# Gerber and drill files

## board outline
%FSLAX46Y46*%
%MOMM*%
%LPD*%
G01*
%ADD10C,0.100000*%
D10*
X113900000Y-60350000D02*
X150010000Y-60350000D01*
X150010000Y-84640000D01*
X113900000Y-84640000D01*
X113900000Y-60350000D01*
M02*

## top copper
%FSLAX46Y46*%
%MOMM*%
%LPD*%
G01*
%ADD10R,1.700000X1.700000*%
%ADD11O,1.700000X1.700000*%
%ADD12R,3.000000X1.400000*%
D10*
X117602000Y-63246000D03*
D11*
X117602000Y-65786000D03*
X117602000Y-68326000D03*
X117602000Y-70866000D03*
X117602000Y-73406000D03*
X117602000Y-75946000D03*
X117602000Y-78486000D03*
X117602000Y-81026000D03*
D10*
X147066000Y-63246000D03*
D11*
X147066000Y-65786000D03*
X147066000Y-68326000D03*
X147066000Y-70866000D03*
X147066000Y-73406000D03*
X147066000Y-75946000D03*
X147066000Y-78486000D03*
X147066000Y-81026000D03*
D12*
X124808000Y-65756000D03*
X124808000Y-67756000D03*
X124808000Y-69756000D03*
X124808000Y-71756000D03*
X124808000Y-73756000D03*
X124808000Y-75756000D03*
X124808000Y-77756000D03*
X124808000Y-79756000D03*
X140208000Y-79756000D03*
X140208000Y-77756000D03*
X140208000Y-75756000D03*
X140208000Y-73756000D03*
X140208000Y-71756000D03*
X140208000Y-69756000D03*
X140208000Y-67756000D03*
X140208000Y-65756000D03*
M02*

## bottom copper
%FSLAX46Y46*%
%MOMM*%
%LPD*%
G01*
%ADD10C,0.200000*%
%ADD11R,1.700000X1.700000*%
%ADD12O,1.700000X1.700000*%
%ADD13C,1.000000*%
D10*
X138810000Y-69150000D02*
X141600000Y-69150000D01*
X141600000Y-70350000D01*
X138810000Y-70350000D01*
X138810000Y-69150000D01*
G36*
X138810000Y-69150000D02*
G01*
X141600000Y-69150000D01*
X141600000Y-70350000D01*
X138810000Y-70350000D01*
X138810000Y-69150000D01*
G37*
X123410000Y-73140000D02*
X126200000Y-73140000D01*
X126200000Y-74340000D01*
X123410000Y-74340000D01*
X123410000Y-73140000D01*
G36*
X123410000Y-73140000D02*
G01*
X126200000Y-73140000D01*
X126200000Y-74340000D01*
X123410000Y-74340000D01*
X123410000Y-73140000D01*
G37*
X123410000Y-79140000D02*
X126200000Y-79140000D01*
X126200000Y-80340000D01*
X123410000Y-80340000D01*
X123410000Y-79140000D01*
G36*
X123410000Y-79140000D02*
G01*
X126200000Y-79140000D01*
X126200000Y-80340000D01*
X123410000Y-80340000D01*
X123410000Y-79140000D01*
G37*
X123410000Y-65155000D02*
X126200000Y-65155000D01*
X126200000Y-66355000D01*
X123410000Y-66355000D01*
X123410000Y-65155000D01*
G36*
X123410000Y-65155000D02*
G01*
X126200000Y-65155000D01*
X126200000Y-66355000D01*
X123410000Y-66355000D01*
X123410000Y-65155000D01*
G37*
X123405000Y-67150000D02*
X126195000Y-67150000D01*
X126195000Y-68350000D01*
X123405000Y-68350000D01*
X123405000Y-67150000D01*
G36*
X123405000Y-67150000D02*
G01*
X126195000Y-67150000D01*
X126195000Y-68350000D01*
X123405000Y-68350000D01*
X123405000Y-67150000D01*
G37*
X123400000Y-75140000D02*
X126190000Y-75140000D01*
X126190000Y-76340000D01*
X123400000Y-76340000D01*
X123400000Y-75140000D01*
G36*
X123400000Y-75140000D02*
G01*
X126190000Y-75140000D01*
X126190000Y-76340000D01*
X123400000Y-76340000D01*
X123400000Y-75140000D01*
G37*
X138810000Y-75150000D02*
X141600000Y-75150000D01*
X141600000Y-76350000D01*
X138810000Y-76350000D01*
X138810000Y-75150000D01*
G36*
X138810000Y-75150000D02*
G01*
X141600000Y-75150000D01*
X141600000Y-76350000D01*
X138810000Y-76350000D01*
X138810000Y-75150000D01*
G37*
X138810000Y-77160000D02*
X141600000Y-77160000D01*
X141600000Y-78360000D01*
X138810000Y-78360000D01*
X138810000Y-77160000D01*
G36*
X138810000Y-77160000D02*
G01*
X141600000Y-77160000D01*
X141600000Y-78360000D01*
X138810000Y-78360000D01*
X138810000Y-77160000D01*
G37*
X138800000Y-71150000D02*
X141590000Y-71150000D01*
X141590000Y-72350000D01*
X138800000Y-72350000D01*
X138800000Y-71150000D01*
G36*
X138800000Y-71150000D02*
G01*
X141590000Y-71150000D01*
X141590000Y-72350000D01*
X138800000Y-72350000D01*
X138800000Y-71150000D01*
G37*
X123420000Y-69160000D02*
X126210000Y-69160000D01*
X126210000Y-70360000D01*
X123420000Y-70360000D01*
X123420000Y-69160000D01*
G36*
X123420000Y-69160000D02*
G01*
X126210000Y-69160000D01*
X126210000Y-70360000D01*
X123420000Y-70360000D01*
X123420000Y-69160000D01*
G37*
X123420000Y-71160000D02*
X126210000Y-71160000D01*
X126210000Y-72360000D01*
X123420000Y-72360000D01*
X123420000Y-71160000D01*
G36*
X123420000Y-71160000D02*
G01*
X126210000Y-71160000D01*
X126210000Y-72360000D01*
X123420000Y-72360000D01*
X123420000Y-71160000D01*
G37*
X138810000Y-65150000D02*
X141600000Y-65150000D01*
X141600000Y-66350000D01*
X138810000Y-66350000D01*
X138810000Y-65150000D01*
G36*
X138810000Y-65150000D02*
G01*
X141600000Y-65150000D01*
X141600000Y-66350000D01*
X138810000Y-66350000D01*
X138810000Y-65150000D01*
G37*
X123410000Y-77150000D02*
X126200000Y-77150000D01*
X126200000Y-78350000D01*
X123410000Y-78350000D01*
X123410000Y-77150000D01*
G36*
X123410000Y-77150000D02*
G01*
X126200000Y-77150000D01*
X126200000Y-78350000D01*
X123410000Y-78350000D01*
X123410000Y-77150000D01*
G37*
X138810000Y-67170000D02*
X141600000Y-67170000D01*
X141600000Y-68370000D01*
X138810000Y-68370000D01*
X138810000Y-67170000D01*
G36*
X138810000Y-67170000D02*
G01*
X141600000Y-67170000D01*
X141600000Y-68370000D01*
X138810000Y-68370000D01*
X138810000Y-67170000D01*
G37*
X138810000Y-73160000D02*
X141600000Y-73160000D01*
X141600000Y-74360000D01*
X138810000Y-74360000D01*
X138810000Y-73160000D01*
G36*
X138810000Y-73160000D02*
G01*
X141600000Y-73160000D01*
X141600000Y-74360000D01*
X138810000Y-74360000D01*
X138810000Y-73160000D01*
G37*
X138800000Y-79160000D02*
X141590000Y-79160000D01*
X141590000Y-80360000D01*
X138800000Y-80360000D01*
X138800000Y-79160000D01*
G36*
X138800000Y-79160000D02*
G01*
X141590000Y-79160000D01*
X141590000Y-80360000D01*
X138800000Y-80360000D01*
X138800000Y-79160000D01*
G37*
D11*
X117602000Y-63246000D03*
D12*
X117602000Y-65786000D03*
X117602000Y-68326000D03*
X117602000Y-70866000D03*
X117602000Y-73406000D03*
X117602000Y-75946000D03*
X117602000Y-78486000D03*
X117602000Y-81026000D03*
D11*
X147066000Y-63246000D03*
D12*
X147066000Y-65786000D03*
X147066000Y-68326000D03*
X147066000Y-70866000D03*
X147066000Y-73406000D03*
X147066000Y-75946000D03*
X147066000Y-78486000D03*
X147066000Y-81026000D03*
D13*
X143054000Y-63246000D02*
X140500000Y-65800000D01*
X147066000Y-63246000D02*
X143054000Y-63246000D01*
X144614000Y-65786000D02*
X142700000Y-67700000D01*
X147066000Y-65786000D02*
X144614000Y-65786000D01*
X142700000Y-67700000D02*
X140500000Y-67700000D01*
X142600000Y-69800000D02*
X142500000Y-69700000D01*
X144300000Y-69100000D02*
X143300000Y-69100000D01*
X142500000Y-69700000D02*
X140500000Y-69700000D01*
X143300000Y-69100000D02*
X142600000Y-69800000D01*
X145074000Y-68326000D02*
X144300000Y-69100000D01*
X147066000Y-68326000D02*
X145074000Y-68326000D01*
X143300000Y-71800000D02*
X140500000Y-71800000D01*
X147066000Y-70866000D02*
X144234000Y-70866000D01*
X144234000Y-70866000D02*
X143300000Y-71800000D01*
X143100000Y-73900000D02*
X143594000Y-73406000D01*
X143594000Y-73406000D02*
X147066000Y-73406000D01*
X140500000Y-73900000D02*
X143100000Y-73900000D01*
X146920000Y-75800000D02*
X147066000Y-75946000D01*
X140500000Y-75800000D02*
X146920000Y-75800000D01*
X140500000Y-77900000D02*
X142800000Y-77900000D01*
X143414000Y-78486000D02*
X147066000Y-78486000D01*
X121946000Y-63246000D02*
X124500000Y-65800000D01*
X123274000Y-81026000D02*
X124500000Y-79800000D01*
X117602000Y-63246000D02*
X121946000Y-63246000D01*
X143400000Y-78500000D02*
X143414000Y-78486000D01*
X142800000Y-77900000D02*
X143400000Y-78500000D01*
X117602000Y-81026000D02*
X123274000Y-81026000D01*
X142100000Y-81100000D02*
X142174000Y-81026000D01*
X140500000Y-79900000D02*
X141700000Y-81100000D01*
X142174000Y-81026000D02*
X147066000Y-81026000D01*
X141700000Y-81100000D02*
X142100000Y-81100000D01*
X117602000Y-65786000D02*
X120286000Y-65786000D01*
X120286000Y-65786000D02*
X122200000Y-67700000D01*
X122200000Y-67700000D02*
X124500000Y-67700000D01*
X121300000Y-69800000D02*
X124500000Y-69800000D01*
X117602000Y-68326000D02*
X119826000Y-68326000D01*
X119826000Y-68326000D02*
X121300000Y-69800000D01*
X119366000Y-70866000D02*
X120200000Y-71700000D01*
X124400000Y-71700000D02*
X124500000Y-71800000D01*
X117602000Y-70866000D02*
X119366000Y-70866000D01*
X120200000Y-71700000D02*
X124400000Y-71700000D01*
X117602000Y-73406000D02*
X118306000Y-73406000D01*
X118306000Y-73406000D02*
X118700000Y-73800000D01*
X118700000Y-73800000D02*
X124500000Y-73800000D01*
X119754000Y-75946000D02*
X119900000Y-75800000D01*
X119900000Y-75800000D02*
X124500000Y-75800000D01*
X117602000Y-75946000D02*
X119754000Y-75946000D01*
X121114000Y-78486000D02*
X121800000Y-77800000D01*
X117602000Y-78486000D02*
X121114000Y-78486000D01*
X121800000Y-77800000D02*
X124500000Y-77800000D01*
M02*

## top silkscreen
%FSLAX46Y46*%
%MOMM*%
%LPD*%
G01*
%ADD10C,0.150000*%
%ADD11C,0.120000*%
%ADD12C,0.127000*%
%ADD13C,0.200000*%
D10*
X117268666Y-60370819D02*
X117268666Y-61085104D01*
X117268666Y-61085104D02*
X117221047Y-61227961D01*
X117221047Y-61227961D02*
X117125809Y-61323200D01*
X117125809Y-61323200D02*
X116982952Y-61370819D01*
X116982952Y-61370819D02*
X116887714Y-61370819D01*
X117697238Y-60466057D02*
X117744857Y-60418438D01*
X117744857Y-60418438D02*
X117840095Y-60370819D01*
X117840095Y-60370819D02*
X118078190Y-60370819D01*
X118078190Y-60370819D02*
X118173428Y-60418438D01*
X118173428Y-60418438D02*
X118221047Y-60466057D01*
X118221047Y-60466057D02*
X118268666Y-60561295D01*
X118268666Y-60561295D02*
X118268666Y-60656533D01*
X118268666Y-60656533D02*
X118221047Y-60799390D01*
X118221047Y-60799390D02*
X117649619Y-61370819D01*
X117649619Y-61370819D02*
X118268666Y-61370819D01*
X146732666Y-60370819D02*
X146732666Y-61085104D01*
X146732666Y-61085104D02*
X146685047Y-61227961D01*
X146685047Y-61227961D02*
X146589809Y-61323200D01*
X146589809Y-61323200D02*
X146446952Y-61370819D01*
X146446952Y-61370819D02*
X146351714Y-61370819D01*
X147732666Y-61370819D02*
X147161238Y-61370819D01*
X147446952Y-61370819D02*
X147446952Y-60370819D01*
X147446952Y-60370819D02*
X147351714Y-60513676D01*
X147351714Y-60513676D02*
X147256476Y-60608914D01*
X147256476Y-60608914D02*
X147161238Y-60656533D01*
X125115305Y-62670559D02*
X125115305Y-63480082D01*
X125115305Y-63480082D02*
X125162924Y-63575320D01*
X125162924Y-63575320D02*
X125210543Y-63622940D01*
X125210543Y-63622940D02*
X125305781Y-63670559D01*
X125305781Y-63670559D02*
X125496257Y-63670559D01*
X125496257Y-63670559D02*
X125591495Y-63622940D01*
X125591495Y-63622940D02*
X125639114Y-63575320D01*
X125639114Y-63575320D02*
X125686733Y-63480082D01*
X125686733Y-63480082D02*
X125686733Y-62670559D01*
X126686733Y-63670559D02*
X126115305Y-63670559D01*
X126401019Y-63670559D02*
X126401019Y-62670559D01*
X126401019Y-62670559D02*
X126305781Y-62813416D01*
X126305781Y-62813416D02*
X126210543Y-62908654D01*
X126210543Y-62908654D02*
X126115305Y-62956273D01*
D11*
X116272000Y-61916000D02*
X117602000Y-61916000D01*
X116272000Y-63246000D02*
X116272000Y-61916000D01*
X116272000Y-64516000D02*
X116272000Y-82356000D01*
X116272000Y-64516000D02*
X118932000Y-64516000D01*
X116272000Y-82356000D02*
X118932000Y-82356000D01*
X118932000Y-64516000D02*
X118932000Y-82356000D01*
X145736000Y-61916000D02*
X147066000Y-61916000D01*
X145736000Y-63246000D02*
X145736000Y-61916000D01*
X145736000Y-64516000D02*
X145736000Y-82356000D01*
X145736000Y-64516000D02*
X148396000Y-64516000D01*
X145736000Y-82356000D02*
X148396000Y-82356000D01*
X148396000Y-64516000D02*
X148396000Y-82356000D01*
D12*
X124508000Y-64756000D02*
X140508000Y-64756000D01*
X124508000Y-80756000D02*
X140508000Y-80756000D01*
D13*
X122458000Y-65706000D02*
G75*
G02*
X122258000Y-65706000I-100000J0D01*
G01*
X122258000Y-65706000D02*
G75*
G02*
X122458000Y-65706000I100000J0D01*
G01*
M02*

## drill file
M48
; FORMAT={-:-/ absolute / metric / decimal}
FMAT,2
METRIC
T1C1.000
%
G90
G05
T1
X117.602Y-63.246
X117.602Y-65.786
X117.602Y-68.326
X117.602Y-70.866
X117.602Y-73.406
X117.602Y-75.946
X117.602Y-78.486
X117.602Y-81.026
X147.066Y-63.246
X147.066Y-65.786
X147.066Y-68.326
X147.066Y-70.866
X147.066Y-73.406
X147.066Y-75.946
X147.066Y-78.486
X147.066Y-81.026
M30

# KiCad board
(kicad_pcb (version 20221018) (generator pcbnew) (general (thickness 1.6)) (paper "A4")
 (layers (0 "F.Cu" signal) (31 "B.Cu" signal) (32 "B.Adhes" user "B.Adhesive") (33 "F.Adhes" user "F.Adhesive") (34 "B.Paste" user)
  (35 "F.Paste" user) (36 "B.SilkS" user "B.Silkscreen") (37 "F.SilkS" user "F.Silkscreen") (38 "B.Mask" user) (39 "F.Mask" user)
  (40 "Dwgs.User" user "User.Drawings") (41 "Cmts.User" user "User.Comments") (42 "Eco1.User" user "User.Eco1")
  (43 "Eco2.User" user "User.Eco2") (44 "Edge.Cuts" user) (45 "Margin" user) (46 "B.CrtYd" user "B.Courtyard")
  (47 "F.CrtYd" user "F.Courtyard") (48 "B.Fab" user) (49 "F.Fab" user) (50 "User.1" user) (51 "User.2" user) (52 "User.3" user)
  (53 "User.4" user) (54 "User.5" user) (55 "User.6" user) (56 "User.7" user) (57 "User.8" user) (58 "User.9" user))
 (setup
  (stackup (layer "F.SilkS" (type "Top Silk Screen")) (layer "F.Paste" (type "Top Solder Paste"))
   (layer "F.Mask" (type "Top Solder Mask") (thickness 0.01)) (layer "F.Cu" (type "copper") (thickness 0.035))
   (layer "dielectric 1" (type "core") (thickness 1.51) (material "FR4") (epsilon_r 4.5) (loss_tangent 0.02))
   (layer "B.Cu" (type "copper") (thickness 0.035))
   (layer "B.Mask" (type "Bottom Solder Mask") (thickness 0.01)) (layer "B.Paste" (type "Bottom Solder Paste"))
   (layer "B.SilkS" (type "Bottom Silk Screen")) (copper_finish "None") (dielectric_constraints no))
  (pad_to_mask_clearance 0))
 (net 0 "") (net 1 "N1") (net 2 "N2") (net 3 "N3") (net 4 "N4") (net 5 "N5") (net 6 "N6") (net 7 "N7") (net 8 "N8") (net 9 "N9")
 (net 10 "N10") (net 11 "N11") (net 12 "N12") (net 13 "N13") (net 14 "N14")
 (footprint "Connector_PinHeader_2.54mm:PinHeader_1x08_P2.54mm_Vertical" (layer "F.Cu") (at 117.602 63.246)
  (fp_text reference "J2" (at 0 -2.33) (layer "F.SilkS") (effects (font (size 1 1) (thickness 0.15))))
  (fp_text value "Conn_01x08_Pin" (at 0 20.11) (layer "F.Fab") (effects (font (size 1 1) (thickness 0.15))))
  (fp_line (start -1.33 -1.33) (end 0 -1.33) (stroke (width 0.12) (type solid)) (layer "F.SilkS"))
  (fp_line (start -1.33 0) (end -1.33 -1.33) (stroke (width 0.12) (type solid)) (layer "F.SilkS"))
  (fp_line (start -1.33 1.27) (end -1.33 19.11) (stroke (width 0.12) (type solid)) (layer "F.SilkS"))
  (fp_line (start -1.33 1.27) (end 1.33 1.27) (stroke (width 0.12) (type solid)) (layer "F.SilkS"))
  (fp_line (start -1.33 19.11) (end 1.33 19.11) (stroke (width 0.12) (type solid)) (layer "F.SilkS"))
  (fp_line (start 1.33 1.27) (end 1.33 19.11) (stroke (width 0.12) (type solid)) (layer "F.SilkS"))
  (pad "1" thru_hole rect (at 0 0) (size 1.7 1.7) (drill 1) (layers "*.Cu" "*.Mask") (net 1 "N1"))
  (pad "2" thru_hole oval (at 0 2.54) (size 1.7 1.7) (drill 1) (layers "*.Cu" "*.Mask") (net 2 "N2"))
  (pad "3" thru_hole oval (at 0 5.08) (size 1.7 1.7) (drill 1) (layers "*.Cu" "*.Mask") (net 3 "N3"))
  (pad "4" thru_hole oval (at 0 7.62) (size 1.7 1.7) (drill 1) (layers "*.Cu" "*.Mask") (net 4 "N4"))
  (pad "5" thru_hole oval (at 0 10.16) (size 1.7 1.7) (drill 1) (layers "*.Cu" "*.Mask") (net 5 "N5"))
  (pad "6" thru_hole oval (at 0 12.7) (size 1.7 1.7) (drill 1) (layers "*.Cu" "*.Mask") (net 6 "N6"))
  (pad "7" thru_hole oval (at 0 15.24) (size 1.7 1.7) (drill 1) (layers "*.Cu" "*.Mask") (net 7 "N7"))
  (pad "8" thru_hole oval (at 0 17.78) (size 1.7 1.7) (drill 1) (layers "*.Cu" "*.Mask") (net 1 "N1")))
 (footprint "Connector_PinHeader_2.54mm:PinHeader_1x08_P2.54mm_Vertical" (layer "F.Cu") (at 147.066 63.246)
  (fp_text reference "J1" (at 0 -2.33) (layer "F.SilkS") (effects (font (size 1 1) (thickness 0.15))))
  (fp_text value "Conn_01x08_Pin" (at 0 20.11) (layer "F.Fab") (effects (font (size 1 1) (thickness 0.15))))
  (fp_line (start -1.33 -1.33) (end 0 -1.33) (stroke (width 0.12) (type solid)) (layer "F.SilkS"))
  (fp_line (start -1.33 0) (end -1.33 -1.33) (stroke (width 0.12) (type solid)) (layer "F.SilkS"))
  (fp_line (start -1.33 1.27) (end -1.33 19.11) (stroke (width 0.12) (type solid)) (layer "F.SilkS"))
  (fp_line (start -1.33 1.27) (end 1.33 1.27) (stroke (width 0.12) (type solid)) (layer "F.SilkS"))
  (fp_line (start -1.33 19.11) (end 1.33 19.11) (stroke (width 0.12) (type solid)) (layer "F.SilkS"))
  (fp_line (start 1.33 1.27) (end 1.33 19.11) (stroke (width 0.12) (type solid)) (layer "F.SilkS"))
  (pad "1" thru_hole rect (at 0 0) (size 1.7 1.7) (drill 1) (layers "*.Cu" "*.Mask") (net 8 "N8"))
  (pad "2" thru_hole oval (at 0 2.54) (size 1.7 1.7) (drill 1) (layers "*.Cu" "*.Mask") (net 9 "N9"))
  (pad "3" thru_hole oval (at 0 5.08) (size 1.7 1.7) (drill 1) (layers "*.Cu" "*.Mask") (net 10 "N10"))
  (pad "4" thru_hole oval (at 0 7.62) (size 1.7 1.7) (drill 1) (layers "*.Cu" "*.Mask") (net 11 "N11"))
  (pad "5" thru_hole oval (at 0 10.16) (size 1.7 1.7) (drill 1) (layers "*.Cu" "*.Mask") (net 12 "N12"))
  (pad "6" thru_hole oval (at 0 12.7) (size 1.7 1.7) (drill 1) (layers "*.Cu" "*.Mask") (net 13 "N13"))
  (pad "7" thru_hole oval (at 0 15.24) (size 1.7 1.7) (drill 1) (layers "*.Cu" "*.Mask") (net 1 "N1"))
  (pad "8" thru_hole oval (at 0 17.78) (size 1.7 1.7) (drill 1) (layers "*.Cu" "*.Mask") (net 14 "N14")))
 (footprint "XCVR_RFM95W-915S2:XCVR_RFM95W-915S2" (layer "F.Cu") (at 132.508 72.756)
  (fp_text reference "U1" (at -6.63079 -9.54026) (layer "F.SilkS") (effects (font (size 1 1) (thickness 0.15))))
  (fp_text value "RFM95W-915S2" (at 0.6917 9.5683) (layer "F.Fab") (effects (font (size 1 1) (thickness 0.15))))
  (fp_line (start -8 -8) (end 8 -8) (stroke (width 0.127) (type solid)) (layer "F.SilkS"))
  (fp_line (start -8 8) (end 8 8) (stroke (width 0.127) (type solid)) (layer "F.SilkS"))
  (fp_circle (center -10.15 -7.05) (end -10.05 -7.05) (stroke (width 0.2) (type solid)) (fill none) (layer "F.SilkS"))
  (pad "1" smd rect (at -7.7 -7) (size 3 1.4) (layers "F.Cu" "F.Paste" "F.Mask") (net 1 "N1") (solder_mask_margin 0.102))
  (pad "2" smd rect (at -7.7 -5) (size 3 1.4) (layers "F.Cu" "F.Paste" "F.Mask") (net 2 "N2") (solder_mask_margin 0.102))
  (pad "3" smd rect (at -7.7 -3) (size 3 1.4) (layers "F.Cu" "F.Paste" "F.Mask") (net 3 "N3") (solder_mask_margin 0.102))
  (pad "4" smd rect (at -7.7 -1) (size 3 1.4) (layers "F.Cu" "F.Paste" "F.Mask") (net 4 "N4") (solder_mask_margin 0.102))
  (pad "5" smd rect (at -7.7 1) (size 3 1.4) (layers "F.Cu" "F.Paste" "F.Mask") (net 5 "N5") (solder_mask_margin 0.102))
  (pad "6" smd rect (at -7.7 3) (size 3 1.4) (layers "F.Cu" "F.Paste" "F.Mask") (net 6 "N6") (solder_mask_margin 0.102))
  (pad "7" smd rect (at -7.7 5) (size 3 1.4) (layers "F.Cu" "F.Paste" "F.Mask") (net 7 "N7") (solder_mask_margin 0.102))
  (pad "8" smd rect (at -7.7 7) (size 3 1.4) (layers "F.Cu" "F.Paste" "F.Mask") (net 1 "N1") (solder_mask_margin 0.102))
  (pad "9" smd rect (at 7.7 7) (size 3 1.4) (layers "F.Cu" "F.Paste" "F.Mask") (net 14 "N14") (solder_mask_margin 0.102))
  (pad "10" smd rect (at 7.7 5) (size 3 1.4) (layers "F.Cu" "F.Paste" "F.Mask") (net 1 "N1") (solder_mask_margin 0.102))
  (pad "11" smd rect (at 7.7 3) (size 3 1.4) (layers "F.Cu" "F.Paste" "F.Mask") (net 13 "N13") (solder_mask_margin 0.102))
  (pad "12" smd rect (at 7.7 1) (size 3 1.4) (layers "F.Cu" "F.Paste" "F.Mask") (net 12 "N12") (solder_mask_margin 0.102))
  (pad "13" smd rect (at 7.7 -1) (size 3 1.4) (layers "F.Cu" "F.Paste" "F.Mask") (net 11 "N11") (solder_mask_margin 0.102))
  (pad "14" smd rect (at 7.7 -3) (size 3 1.4) (layers "F.Cu" "F.Paste" "F.Mask") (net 10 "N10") (solder_mask_margin 0.102))
  (pad "15" smd rect (at 7.7 -5) (size 3 1.4) (layers "F.Cu" "F.Paste" "F.Mask") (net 9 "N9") (solder_mask_margin 0.102))
  (pad "16" smd rect (at 7.7 -7) (size 3 1.4) (layers "F.Cu" "F.Paste" "F.Mask") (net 8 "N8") (solder_mask_margin 0.102)))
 (gr_rect (start 138.81 69.15) (end 141.6 70.35) (stroke (width 0.2) (type solid)) (fill solid) (layer "B.Cu"))
 (gr_rect (start 123.41 73.14) (end 126.2 74.34) (stroke (width 0.2) (type solid)) (fill solid) (layer "B.Cu"))
 (gr_rect (start 123.41 79.14) (end 126.2 80.34) (stroke (width 0.2) (type solid)) (fill solid) (layer "B.Cu"))
 (gr_rect (start 123.41 65.155) (end 126.2 66.355) (stroke (width 0.2) (type solid)) (fill solid) (layer "B.Cu"))
 (gr_rect (start 123.405 67.15) (end 126.195 68.35) (stroke (width 0.2) (type solid)) (fill solid) (layer "B.Cu"))
 (gr_rect (start 123.4 75.14) (end 126.19 76.34) (stroke (width 0.2) (type solid)) (fill solid) (layer "B.Cu"))
 (gr_rect (start 138.81 75.15) (end 141.6 76.35) (stroke (width 0.2) (type solid)) (fill solid) (layer "B.Cu"))
 (gr_rect (start 138.81 77.16) (end 141.6 78.36) (stroke (width 0.2) (type solid)) (fill solid) (layer "B.Cu"))
 (gr_rect (start 138.8 71.15) (end 141.59 72.35) (stroke (width 0.2) (type solid)) (fill solid) (layer "B.Cu"))
 (gr_rect (start 123.42 69.16) (end 126.21 70.36) (stroke (width 0.2) (type solid)) (fill solid) (layer "B.Cu"))
 (gr_rect (start 123.42 71.16) (end 126.21 72.36) (stroke (width 0.2) (type solid)) (fill solid) (layer "B.Cu"))
 (gr_rect (start 138.81 65.15) (end 141.6 66.35) (stroke (width 0.2) (type solid)) (fill solid) (layer "B.Cu"))
 (gr_rect (start 123.41 77.15) (end 126.2 78.35) (stroke (width 0.2) (type solid)) (fill solid) (layer "B.Cu"))
 (gr_rect (start 138.81 67.17) (end 141.6 68.37) (stroke (width 0.2) (type solid)) (fill solid) (layer "B.Cu"))
 (gr_rect (start 138.81 73.16) (end 141.6 74.36) (stroke (width 0.2) (type solid)) (fill solid) (layer "B.Cu"))
 (gr_rect (start 138.8 79.16) (end 141.59 80.36) (stroke (width 0.2) (type solid)) (fill solid) (layer "B.Cu"))
 (gr_rect (start 113.9 60.35) (end 150.01 84.64) (stroke (width 0.1) (type default)) (fill none) (layer "Edge.Cuts"))
 (segment (start 143.054 63.246) (end 140.5 65.8) (width 1) (layer "B.Cu") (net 8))
 (segment (start 147.066 63.246) (end 143.054 63.246) (width 1) (layer "B.Cu") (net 8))
 (segment (start 144.614 65.786) (end 142.7 67.7) (width 1) (layer "B.Cu") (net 9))
 (segment (start 147.066 65.786) (end 144.614 65.786) (width 1) (layer "B.Cu") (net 9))
 (segment (start 142.7 67.7) (end 140.5 67.7) (width 1) (layer "B.Cu") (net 9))
 (segment (start 142.6 69.8) (end 142.5 69.7) (width 1) (layer "B.Cu") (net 10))
 (segment (start 144.3 69.1) (end 143.3 69.1) (width 1) (layer "B.Cu") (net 10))
 (segment (start 142.5 69.7) (end 140.5 69.7) (width 1) (layer "B.Cu") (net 10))
 (segment (start 143.3 69.1) (end 142.6 69.8) (width 1) (layer "B.Cu") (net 10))
 (segment (start 145.074 68.326) (end 144.3 69.1) (width 1) (layer "B.Cu") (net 10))
 (segment (start 147.066 68.326) (end 145.074 68.326) (width 1) (layer "B.Cu") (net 10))
 (segment (start 143.3 71.8) (end 140.5 71.8) (width 1) (layer "B.Cu") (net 11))
 (segment (start 147.066 70.866) (end 144.234 70.866) (width 1) (layer "B.Cu") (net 11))
 (segment (start 144.234 70.866) (end 143.3 71.8) (width 1) (layer "B.Cu") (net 11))
 (segment (start 143.1 73.9) (end 143.594 73.406) (width 1) (layer "B.Cu") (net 12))
 (segment (start 143.594 73.406) (end 147.066 73.406) (width 1) (layer "B.Cu") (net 12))
 (segment (start 140.5 73.9) (end 143.1 73.9) (width 1) (layer "B.Cu") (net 12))
 (segment (start 146.92 75.8) (end 147.066 75.946) (width 1) (layer "B.Cu") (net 13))
 (segment (start 140.5 75.8) (end 146.92 75.8) (width 1) (layer "B.Cu") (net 13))
 (segment (start 140.5 77.9) (end 142.8 77.9) (width 1) (layer "B.Cu") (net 1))
 (segment (start 143.414 78.486) (end 147.066 78.486) (width 1) (layer "B.Cu") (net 1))
 (segment (start 121.946 63.246) (end 124.5 65.8) (width 1) (layer "B.Cu") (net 1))
 (segment (start 123.274 81.026) (end 124.5 79.8) (width 1) (layer "B.Cu") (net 1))
 (segment (start 117.602 63.246) (end 121.946 63.246) (width 1) (layer "B.Cu") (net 1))
 (segment (start 143.4 78.5) (end 143.414 78.486) (width 1) (layer "B.Cu") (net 1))
 (segment (start 142.8 77.9) (end 143.4 78.5) (width 1) (layer "B.Cu") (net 1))
 (segment (start 117.602 81.026) (end 123.274 81.026) (width 1) (layer "B.Cu") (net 1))
 (segment (start 142.1 81.1) (end 142.174 81.026) (width 1) (layer "B.Cu") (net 14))
 (segment (start 140.5 79.9) (end 141.7 81.1) (width 1) (layer "B.Cu") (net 14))
 (segment (start 142.174 81.026) (end 147.066 81.026) (width 1) (layer "B.Cu") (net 14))
 (segment (start 141.7 81.1) (end 142.1 81.1) (width 1) (layer "B.Cu") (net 14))
 (segment (start 117.602 65.786) (end 120.286 65.786) (width 1) (layer "B.Cu") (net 2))
 (segment (start 120.286 65.786) (end 122.2 67.7) (width 1) (layer "B.Cu") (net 2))
 (segment (start 122.2 67.7) (end 124.5 67.7) (width 1) (layer "B.Cu") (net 2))
 (segment (start 121.3 69.8) (end 124.5 69.8) (width 1) (layer "B.Cu") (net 3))
 (segment (start 117.602 68.326) (end 119.826 68.326) (width 1) (layer "B.Cu") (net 3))
 (segment (start 119.826 68.326) (end 121.3 69.8) (width 1) (layer "B.Cu") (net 3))
 (segment (start 119.366 70.866) (end 120.2 71.7) (width 1) (layer "B.Cu") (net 4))
 (segment (start 124.4 71.7) (end 124.5 71.8) (width 1) (layer "B.Cu") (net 4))
 (segment (start 117.602 70.866) (end 119.366 70.866) (width 1) (layer "B.Cu") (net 4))
 (segment (start 120.2 71.7) (end 124.4 71.7) (width 1) (layer "B.Cu") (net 4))
 (segment (start 117.602 73.406) (end 118.306 73.406) (width 1) (layer "B.Cu") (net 5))
 (segment (start 118.306 73.406) (end 118.7 73.8) (width 1) (layer "B.Cu") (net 5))
 (segment (start 118.7 73.8) (end 124.5 73.8) (width 1) (layer "B.Cu") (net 5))
 (segment (start 119.754 75.946) (end 119.9 75.8) (width 1) (layer "B.Cu") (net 6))
 (segment (start 119.9 75.8) (end 124.5 75.8) (width 1) (layer "B.Cu") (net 6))
 (segment (start 117.602 75.946) (end 119.754 75.946) (width 1) (layer "B.Cu") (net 6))
 (segment (start 121.114 78.486) (end 121.8 77.8) (width 1) (layer "B.Cu") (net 7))
 (segment (start 117.602 78.486) (end 121.114 78.486) (width 1) (layer "B.Cu") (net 7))
 (segment (start 121.8 77.8) (end 124.5 77.8) (width 1) (layer "B.Cu") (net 7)))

